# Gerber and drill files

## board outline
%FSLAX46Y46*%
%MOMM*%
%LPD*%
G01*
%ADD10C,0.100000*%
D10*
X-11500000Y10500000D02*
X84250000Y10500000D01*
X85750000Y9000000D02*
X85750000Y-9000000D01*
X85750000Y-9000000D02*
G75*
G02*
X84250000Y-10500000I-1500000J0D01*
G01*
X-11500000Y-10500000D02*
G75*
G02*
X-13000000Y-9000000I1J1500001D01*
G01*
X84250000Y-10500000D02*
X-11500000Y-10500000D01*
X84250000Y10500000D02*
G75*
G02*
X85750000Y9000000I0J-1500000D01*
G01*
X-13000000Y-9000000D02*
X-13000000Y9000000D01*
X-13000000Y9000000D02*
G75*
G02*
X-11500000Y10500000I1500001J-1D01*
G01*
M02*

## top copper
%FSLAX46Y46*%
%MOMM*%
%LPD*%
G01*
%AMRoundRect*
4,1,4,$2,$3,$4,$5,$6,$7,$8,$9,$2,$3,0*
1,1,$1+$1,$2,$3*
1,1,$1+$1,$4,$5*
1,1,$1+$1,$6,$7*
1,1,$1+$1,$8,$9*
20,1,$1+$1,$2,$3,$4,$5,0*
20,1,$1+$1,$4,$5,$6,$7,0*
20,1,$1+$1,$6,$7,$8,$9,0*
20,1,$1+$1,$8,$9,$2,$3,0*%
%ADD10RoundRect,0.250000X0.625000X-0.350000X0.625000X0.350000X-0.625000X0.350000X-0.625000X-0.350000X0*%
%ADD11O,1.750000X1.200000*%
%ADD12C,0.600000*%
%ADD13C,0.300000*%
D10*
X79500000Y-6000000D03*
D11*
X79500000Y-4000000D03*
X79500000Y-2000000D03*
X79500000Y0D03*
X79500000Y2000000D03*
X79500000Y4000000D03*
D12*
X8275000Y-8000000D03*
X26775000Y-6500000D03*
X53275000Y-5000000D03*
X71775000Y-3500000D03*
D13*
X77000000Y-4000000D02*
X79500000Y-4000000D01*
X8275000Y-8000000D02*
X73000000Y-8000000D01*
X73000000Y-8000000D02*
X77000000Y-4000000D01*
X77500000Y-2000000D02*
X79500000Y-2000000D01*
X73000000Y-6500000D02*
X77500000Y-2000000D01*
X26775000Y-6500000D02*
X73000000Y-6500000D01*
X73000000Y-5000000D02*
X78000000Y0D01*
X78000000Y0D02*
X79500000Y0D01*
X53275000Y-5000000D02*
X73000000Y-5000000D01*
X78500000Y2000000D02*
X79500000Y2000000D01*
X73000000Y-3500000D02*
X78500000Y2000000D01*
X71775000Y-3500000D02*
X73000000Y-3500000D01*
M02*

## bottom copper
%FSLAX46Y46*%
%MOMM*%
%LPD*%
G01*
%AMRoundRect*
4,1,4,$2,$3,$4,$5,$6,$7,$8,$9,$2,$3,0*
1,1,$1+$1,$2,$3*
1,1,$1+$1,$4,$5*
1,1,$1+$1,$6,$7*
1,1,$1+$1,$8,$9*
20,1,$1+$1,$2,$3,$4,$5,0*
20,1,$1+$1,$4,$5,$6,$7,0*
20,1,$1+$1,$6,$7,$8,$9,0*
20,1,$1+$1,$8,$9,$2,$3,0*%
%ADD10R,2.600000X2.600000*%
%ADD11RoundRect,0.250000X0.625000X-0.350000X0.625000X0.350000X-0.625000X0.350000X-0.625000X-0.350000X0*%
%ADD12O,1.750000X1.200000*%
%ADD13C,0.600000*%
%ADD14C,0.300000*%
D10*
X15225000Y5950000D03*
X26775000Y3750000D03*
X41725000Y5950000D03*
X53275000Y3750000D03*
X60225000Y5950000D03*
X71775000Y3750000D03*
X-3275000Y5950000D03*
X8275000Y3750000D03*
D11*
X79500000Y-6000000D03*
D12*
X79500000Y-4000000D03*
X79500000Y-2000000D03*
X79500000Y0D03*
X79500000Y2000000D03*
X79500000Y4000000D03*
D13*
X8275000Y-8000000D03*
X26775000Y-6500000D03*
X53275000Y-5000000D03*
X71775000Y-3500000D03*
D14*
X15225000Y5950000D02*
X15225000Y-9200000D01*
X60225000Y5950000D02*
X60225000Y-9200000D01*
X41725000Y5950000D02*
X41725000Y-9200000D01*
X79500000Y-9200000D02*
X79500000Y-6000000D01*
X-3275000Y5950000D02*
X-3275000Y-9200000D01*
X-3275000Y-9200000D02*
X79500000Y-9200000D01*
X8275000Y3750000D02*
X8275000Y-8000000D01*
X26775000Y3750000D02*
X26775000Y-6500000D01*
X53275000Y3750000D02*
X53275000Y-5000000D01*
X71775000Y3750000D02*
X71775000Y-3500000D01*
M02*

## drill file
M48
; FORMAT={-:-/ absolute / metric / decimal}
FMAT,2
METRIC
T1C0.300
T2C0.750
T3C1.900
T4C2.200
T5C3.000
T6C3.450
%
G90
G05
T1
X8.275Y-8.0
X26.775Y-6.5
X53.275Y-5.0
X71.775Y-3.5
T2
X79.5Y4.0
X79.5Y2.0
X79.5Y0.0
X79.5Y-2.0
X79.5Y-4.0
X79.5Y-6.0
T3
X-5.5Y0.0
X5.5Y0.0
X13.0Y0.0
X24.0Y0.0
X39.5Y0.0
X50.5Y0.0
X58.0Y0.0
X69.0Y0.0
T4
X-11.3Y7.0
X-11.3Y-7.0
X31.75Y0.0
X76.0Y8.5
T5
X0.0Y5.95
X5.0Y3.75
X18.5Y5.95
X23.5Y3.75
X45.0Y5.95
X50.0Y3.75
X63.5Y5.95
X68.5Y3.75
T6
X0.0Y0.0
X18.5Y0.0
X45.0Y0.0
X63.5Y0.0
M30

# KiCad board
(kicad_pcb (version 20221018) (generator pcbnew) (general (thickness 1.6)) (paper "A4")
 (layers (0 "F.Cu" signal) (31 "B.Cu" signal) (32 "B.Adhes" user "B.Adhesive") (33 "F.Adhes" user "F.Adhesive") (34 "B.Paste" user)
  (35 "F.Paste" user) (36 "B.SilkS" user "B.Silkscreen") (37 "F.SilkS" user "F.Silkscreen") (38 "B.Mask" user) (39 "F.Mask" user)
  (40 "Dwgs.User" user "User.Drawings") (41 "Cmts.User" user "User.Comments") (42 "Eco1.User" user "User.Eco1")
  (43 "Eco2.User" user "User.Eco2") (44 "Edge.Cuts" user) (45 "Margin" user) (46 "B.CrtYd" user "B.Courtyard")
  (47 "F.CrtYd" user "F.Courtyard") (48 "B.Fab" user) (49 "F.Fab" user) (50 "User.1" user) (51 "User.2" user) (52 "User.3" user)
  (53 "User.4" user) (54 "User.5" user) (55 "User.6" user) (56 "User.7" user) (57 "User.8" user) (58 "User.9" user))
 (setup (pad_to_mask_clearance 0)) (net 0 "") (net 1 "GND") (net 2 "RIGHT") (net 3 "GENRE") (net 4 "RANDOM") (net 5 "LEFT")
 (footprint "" (layer "F.Cu") (at 31.75 0)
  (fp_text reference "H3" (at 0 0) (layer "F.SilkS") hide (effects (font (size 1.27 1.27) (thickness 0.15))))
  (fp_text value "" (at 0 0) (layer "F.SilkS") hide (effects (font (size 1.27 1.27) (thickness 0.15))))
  (pad "" np_thru_hole circle (at 0 0) (size 2.2 2.2) (drill 2.2) (layers "F&B.Cu" "*.Mask")))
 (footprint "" (layer "F.Cu") (at -11.3 7)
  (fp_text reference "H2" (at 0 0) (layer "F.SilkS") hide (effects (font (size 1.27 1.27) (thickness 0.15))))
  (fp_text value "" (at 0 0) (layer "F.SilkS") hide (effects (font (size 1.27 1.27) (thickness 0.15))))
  (pad "" np_thru_hole circle (at 0 0) (size 2.2 2.2) (drill 2.2) (layers "F&B.Cu" "*.Mask")))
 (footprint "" (layer "F.Cu") (at 18.5 0)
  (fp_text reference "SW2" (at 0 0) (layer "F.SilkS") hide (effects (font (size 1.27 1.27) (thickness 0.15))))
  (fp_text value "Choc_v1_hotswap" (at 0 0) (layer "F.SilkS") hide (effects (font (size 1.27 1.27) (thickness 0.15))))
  (pad "" np_thru_hole circle (at -5.5 0) (size 1.9 1.9) (drill 1.9) (layers "F&B.Cu" "*.Mask"))
  (pad "" np_thru_hole circle (at 0 -5.95) (size 3 3) (drill 3) (layers "F&B.Cu" "*.Mask"))
  (pad "" np_thru_hole circle (at 0 0) (size 3.45 3.45) (drill 3.45) (layers "F&B.Cu" "*.Mask"))
  (pad "" np_thru_hole circle (at 5 -3.75) (size 3 3) (drill 3) (layers "F&B.Cu" "*.Mask"))
  (pad "" np_thru_hole circle (at 5.5 0) (size 1.9 1.9) (drill 1.9) (layers "F&B.Cu" "*.Mask"))
  (pad "1" smd rect (at -3.275 -5.95) (size 2.6 2.6) (layers "B.Cu" "B.Paste" "B.Mask") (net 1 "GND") (thermal_bridge_angle 45))
  (pad "2" smd rect (at 8.275 -3.75) (size 2.6 2.6) (layers "B.Cu" "B.Paste" "B.Mask") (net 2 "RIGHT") (thermal_bridge_angle 45)))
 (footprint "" (layer "F.Cu") (at 45 0)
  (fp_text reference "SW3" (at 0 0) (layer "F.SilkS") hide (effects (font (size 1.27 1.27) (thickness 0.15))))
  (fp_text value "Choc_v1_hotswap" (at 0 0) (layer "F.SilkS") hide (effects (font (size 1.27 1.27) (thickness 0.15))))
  (pad "" np_thru_hole circle (at -5.5 0) (size 1.9 1.9) (drill 1.9) (layers "F&B.Cu" "*.Mask"))
  (pad "" np_thru_hole circle (at 0 -5.95) (size 3 3) (drill 3) (layers "F&B.Cu" "*.Mask"))
  (pad "" np_thru_hole circle (at 0 0) (size 3.45 3.45) (drill 3.45) (layers "F&B.Cu" "*.Mask"))
  (pad "" np_thru_hole circle (at 5 -3.75) (size 3 3) (drill 3) (layers "F&B.Cu" "*.Mask"))
  (pad "" np_thru_hole circle (at 5.5 0) (size 1.9 1.9) (drill 1.9) (layers "F&B.Cu" "*.Mask"))
  (pad "1" smd rect (at -3.275 -5.95) (size 2.6 2.6) (layers "B.Cu" "B.Paste" "B.Mask") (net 1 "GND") (thermal_bridge_angle 45))
  (pad "2" smd rect (at 8.275 -3.75) (size 2.6 2.6) (layers "B.Cu" "B.Paste" "B.Mask") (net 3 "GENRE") (thermal_bridge_angle 45)))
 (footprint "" (layer "F.Cu") (at 63.5 0)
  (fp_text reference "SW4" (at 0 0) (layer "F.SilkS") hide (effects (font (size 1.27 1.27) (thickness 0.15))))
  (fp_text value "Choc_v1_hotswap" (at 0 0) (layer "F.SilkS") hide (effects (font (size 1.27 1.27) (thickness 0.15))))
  (pad "" np_thru_hole circle (at -5.5 0) (size 1.9 1.9) (drill 1.9) (layers "F&B.Cu" "*.Mask"))
  (pad "" np_thru_hole circle (at 0 -5.95) (size 3 3) (drill 3) (layers "F&B.Cu" "*.Mask"))
  (pad "" np_thru_hole circle (at 0 0) (size 3.45 3.45) (drill 3.45) (layers "F&B.Cu" "*.Mask"))
  (pad "" np_thru_hole circle (at 5 -3.75) (size 3 3) (drill 3) (layers "F&B.Cu" "*.Mask"))
  (pad "" np_thru_hole circle (at 5.5 0) (size 1.9 1.9) (drill 1.9) (layers "F&B.Cu" "*.Mask"))
  (pad "1" smd rect (at -3.275 -5.95) (size 2.6 2.6) (layers "B.Cu" "B.Paste" "B.Mask") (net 1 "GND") (thermal_bridge_angle 45))
  (pad "2" smd rect (at 8.275 -3.75) (size 2.6 2.6) (layers "B.Cu" "B.Paste" "B.Mask") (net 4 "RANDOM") (thermal_bridge_angle 45)))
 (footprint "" (layer "F.Cu") (at 76 -8.5)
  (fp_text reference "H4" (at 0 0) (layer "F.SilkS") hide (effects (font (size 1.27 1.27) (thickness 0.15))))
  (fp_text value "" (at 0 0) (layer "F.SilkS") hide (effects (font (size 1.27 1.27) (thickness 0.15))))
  (pad "" np_thru_hole circle (at 0 0) (size 2.2 2.2) (drill 2.2) (layers "F&B.Cu" "*.Mask")))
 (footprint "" (layer "F.Cu") (at 0 0)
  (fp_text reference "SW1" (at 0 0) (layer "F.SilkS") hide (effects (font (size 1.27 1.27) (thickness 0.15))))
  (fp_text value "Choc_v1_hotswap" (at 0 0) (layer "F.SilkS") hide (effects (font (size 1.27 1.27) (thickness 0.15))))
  (pad "" np_thru_hole circle (at -5.5 0) (size 1.9 1.9) (drill 1.9) (layers "F&B.Cu" "*.Mask"))
  (pad "" np_thru_hole circle (at 0 -5.95) (size 3 3) (drill 3) (layers "F&B.Cu" "*.Mask"))
  (pad "" np_thru_hole circle (at 0 0) (size 3.45 3.45) (drill 3.45) (layers "F&B.Cu" "*.Mask"))
  (pad "" np_thru_hole circle (at 5 -3.75) (size 3 3) (drill 3) (layers "F&B.Cu" "*.Mask"))
  (pad "" np_thru_hole circle (at 5.5 0) (size 1.9 1.9) (drill 1.9) (layers "F&B.Cu" "*.Mask"))
  (pad "1" smd rect (at -3.275 -5.95) (size 2.6 2.6) (layers "B.Cu" "B.Paste" "B.Mask") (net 1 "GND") (thermal_bridge_angle 45))
  (pad "2" smd rect (at 8.275 -3.75) (size 2.6 2.6) (layers "B.Cu" "B.Paste" "B.Mask") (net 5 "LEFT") (thermal_bridge_angle 45)))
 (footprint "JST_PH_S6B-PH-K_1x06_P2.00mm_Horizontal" (layer "F.Cu") (at 79.5 6 90)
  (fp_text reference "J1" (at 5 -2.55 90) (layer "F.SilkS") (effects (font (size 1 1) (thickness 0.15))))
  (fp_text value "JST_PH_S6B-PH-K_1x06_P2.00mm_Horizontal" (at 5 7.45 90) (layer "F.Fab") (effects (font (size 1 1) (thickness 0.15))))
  (pad "1" thru_hole roundrect (at 0 0 90) (size 1.2 1.75) (drill 0.75) (layers "*.Cu" "*.Mask") (roundrect_rratio 0.208333) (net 1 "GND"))
  (pad "2" thru_hole oval (at 2 0 90) (size 1.2 1.75) (drill 0.75) (layers "*.Cu" "*.Mask") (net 5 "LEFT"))
  (pad "3" thru_hole oval (at 4 0 90) (size 1.2 1.75) (drill 0.75) (layers "*.Cu" "*.Mask") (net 2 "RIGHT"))
  (pad "4" thru_hole oval (at 6 0 90) (size 1.2 1.75) (drill 0.75) (layers "*.Cu" "*.Mask") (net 3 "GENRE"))
  (pad "5" thru_hole oval (at 8 0 90) (size 1.2 1.75) (drill 0.75) (layers "*.Cu" "*.Mask") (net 4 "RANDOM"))
  (pad "6" thru_hole oval (at 10 0 90) (size 1.2 1.75) (drill 0.75) (layers "*.Cu" "*.Mask")))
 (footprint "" (layer "F.Cu") (at -11.3 -7)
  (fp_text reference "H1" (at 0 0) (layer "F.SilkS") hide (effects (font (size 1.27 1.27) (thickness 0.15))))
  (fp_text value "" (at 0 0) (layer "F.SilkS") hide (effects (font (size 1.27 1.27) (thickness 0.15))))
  (pad "" np_thru_hole circle (at 0 0) (size 2.2 2.2) (drill 2.2) (layers "F&B.Cu" "*.Mask")))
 (gr_line (start -11.5 -10.5) (end 84.25 -10.5) (stroke (width 0.1) (type default)) (layer "Edge.Cuts"))
 (gr_line (start 85.75 -9) (end 85.75 9) (stroke (width 0.1) (type default)) (layer "Edge.Cuts"))
 (gr_arc (start 85.75 9) (mid 85.31066 10.06066) (end 84.25 10.5) (stroke (width 0.1) (type default)) (layer "Edge.Cuts"))
 (gr_arc (start -11.5 10.5) (mid -12.56066 10.06066) (end -13 9) (stroke (width 0.1) (type default)) (layer "Edge.Cuts"))
 (gr_line (start 84.25 10.5) (end -11.5 10.5) (stroke (width 0.1) (type default)) (layer "Edge.Cuts"))
 (gr_arc (start 84.25 -10.5) (mid 85.31066 -10.06066) (end 85.75 -9) (stroke (width 0.1) (type default)) (layer "Edge.Cuts"))
 (gr_line (start -13 9) (end -13 -9) (stroke (width 0.1) (type default)) (layer "Edge.Cuts"))
 (gr_arc (start -13 -9) (mid -12.56066 -10.06066) (end -11.5 -10.5) (stroke (width 0.1) (type default)) (layer "Edge.Cuts"))
 (segment (start 15.225 -5.95) (end 15.225 9.2) (width 0.3) (layer "B.Cu") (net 1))
 (segment (start 60.225 -5.95) (end 60.225 9.2) (width 0.3) (layer "B.Cu") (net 1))
 (segment (start 41.725 -5.95) (end 41.725 9.2) (width 0.3) (layer "B.Cu") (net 1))
 (segment (start 79.5 9.2) (end 79.5 6) (width 0.3) (layer "B.Cu") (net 1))
 (segment (start -3.275 -5.95) (end -3.275 9.2) (width 0.3) (layer "B.Cu") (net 1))
 (segment (start -3.275 9.2) (end 79.5 9.2) (width 0.3) (layer "B.Cu") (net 1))
 (segment (start 77 4) (end 79.5 4) (width 0.3) (layer "F.Cu") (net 5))
 (segment (start 8.275 8) (end 73 8) (width 0.3) (layer "F.Cu") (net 5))
 (segment (start 73 8) (end 77 4) (width 0.3) (layer "F.Cu") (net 5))
 (via (at 8.275 8) (size 0.6) (drill 0.3) (layers "F.Cu" "B.Cu") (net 5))
 (segment (start 8.275 -3.75) (end 8.275 8) (width 0.3) (layer "B.Cu") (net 5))
 (segment (start 77.5 2) (end 79.5 2) (width 0.3) (layer "F.Cu") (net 2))
 (segment (start 73 6.5) (end 77.5 2) (width 0.3) (layer "F.Cu") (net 2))
 (segment (start 26.775 6.5) (end 73 6.5) (width 0.3) (layer "F.Cu") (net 2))
 (via (at 26.775 6.5) (size 0.6) (drill 0.3) (layers "F.Cu" "B.Cu") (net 2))
 (segment (start 26.775 -3.75) (end 26.775 6.5) (width 0.3) (layer "B.Cu") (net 2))
 (segment (start 73 5) (end 78 0) (width 0.3) (layer "F.Cu") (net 3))
 (segment (start 78 0) (end 79.5 0) (width 0.3) (layer "F.Cu") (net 3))
 (segment (start 53.275 5) (end 73 5) (width 0.3) (layer "F.Cu") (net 3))
 (via (at 53.275 5) (size 0.6) (drill 0.3) (layers "F.Cu" "B.Cu") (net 3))
 (segment (start 53.275 -3.75) (end 53.275 5) (width 0.3) (layer "B.Cu") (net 3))
 (segment (start 78.5 -2) (end 79.5 -2) (width 0.3) (layer "F.Cu") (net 4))
 (segment (start 73 3.5) (end 78.5 -2) (width 0.3) (layer "F.Cu") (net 4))
 (segment (start 71.775 3.5) (end 73 3.5) (width 0.3) (layer "F.Cu") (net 4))
 (via (at 71.775 3.5) (size 0.6) (drill 0.3) (layers "F.Cu" "B.Cu") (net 4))
 (segment (start 71.775 -3.75) (end 71.775 3.5) (width 0.3) (layer "B.Cu") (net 4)))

